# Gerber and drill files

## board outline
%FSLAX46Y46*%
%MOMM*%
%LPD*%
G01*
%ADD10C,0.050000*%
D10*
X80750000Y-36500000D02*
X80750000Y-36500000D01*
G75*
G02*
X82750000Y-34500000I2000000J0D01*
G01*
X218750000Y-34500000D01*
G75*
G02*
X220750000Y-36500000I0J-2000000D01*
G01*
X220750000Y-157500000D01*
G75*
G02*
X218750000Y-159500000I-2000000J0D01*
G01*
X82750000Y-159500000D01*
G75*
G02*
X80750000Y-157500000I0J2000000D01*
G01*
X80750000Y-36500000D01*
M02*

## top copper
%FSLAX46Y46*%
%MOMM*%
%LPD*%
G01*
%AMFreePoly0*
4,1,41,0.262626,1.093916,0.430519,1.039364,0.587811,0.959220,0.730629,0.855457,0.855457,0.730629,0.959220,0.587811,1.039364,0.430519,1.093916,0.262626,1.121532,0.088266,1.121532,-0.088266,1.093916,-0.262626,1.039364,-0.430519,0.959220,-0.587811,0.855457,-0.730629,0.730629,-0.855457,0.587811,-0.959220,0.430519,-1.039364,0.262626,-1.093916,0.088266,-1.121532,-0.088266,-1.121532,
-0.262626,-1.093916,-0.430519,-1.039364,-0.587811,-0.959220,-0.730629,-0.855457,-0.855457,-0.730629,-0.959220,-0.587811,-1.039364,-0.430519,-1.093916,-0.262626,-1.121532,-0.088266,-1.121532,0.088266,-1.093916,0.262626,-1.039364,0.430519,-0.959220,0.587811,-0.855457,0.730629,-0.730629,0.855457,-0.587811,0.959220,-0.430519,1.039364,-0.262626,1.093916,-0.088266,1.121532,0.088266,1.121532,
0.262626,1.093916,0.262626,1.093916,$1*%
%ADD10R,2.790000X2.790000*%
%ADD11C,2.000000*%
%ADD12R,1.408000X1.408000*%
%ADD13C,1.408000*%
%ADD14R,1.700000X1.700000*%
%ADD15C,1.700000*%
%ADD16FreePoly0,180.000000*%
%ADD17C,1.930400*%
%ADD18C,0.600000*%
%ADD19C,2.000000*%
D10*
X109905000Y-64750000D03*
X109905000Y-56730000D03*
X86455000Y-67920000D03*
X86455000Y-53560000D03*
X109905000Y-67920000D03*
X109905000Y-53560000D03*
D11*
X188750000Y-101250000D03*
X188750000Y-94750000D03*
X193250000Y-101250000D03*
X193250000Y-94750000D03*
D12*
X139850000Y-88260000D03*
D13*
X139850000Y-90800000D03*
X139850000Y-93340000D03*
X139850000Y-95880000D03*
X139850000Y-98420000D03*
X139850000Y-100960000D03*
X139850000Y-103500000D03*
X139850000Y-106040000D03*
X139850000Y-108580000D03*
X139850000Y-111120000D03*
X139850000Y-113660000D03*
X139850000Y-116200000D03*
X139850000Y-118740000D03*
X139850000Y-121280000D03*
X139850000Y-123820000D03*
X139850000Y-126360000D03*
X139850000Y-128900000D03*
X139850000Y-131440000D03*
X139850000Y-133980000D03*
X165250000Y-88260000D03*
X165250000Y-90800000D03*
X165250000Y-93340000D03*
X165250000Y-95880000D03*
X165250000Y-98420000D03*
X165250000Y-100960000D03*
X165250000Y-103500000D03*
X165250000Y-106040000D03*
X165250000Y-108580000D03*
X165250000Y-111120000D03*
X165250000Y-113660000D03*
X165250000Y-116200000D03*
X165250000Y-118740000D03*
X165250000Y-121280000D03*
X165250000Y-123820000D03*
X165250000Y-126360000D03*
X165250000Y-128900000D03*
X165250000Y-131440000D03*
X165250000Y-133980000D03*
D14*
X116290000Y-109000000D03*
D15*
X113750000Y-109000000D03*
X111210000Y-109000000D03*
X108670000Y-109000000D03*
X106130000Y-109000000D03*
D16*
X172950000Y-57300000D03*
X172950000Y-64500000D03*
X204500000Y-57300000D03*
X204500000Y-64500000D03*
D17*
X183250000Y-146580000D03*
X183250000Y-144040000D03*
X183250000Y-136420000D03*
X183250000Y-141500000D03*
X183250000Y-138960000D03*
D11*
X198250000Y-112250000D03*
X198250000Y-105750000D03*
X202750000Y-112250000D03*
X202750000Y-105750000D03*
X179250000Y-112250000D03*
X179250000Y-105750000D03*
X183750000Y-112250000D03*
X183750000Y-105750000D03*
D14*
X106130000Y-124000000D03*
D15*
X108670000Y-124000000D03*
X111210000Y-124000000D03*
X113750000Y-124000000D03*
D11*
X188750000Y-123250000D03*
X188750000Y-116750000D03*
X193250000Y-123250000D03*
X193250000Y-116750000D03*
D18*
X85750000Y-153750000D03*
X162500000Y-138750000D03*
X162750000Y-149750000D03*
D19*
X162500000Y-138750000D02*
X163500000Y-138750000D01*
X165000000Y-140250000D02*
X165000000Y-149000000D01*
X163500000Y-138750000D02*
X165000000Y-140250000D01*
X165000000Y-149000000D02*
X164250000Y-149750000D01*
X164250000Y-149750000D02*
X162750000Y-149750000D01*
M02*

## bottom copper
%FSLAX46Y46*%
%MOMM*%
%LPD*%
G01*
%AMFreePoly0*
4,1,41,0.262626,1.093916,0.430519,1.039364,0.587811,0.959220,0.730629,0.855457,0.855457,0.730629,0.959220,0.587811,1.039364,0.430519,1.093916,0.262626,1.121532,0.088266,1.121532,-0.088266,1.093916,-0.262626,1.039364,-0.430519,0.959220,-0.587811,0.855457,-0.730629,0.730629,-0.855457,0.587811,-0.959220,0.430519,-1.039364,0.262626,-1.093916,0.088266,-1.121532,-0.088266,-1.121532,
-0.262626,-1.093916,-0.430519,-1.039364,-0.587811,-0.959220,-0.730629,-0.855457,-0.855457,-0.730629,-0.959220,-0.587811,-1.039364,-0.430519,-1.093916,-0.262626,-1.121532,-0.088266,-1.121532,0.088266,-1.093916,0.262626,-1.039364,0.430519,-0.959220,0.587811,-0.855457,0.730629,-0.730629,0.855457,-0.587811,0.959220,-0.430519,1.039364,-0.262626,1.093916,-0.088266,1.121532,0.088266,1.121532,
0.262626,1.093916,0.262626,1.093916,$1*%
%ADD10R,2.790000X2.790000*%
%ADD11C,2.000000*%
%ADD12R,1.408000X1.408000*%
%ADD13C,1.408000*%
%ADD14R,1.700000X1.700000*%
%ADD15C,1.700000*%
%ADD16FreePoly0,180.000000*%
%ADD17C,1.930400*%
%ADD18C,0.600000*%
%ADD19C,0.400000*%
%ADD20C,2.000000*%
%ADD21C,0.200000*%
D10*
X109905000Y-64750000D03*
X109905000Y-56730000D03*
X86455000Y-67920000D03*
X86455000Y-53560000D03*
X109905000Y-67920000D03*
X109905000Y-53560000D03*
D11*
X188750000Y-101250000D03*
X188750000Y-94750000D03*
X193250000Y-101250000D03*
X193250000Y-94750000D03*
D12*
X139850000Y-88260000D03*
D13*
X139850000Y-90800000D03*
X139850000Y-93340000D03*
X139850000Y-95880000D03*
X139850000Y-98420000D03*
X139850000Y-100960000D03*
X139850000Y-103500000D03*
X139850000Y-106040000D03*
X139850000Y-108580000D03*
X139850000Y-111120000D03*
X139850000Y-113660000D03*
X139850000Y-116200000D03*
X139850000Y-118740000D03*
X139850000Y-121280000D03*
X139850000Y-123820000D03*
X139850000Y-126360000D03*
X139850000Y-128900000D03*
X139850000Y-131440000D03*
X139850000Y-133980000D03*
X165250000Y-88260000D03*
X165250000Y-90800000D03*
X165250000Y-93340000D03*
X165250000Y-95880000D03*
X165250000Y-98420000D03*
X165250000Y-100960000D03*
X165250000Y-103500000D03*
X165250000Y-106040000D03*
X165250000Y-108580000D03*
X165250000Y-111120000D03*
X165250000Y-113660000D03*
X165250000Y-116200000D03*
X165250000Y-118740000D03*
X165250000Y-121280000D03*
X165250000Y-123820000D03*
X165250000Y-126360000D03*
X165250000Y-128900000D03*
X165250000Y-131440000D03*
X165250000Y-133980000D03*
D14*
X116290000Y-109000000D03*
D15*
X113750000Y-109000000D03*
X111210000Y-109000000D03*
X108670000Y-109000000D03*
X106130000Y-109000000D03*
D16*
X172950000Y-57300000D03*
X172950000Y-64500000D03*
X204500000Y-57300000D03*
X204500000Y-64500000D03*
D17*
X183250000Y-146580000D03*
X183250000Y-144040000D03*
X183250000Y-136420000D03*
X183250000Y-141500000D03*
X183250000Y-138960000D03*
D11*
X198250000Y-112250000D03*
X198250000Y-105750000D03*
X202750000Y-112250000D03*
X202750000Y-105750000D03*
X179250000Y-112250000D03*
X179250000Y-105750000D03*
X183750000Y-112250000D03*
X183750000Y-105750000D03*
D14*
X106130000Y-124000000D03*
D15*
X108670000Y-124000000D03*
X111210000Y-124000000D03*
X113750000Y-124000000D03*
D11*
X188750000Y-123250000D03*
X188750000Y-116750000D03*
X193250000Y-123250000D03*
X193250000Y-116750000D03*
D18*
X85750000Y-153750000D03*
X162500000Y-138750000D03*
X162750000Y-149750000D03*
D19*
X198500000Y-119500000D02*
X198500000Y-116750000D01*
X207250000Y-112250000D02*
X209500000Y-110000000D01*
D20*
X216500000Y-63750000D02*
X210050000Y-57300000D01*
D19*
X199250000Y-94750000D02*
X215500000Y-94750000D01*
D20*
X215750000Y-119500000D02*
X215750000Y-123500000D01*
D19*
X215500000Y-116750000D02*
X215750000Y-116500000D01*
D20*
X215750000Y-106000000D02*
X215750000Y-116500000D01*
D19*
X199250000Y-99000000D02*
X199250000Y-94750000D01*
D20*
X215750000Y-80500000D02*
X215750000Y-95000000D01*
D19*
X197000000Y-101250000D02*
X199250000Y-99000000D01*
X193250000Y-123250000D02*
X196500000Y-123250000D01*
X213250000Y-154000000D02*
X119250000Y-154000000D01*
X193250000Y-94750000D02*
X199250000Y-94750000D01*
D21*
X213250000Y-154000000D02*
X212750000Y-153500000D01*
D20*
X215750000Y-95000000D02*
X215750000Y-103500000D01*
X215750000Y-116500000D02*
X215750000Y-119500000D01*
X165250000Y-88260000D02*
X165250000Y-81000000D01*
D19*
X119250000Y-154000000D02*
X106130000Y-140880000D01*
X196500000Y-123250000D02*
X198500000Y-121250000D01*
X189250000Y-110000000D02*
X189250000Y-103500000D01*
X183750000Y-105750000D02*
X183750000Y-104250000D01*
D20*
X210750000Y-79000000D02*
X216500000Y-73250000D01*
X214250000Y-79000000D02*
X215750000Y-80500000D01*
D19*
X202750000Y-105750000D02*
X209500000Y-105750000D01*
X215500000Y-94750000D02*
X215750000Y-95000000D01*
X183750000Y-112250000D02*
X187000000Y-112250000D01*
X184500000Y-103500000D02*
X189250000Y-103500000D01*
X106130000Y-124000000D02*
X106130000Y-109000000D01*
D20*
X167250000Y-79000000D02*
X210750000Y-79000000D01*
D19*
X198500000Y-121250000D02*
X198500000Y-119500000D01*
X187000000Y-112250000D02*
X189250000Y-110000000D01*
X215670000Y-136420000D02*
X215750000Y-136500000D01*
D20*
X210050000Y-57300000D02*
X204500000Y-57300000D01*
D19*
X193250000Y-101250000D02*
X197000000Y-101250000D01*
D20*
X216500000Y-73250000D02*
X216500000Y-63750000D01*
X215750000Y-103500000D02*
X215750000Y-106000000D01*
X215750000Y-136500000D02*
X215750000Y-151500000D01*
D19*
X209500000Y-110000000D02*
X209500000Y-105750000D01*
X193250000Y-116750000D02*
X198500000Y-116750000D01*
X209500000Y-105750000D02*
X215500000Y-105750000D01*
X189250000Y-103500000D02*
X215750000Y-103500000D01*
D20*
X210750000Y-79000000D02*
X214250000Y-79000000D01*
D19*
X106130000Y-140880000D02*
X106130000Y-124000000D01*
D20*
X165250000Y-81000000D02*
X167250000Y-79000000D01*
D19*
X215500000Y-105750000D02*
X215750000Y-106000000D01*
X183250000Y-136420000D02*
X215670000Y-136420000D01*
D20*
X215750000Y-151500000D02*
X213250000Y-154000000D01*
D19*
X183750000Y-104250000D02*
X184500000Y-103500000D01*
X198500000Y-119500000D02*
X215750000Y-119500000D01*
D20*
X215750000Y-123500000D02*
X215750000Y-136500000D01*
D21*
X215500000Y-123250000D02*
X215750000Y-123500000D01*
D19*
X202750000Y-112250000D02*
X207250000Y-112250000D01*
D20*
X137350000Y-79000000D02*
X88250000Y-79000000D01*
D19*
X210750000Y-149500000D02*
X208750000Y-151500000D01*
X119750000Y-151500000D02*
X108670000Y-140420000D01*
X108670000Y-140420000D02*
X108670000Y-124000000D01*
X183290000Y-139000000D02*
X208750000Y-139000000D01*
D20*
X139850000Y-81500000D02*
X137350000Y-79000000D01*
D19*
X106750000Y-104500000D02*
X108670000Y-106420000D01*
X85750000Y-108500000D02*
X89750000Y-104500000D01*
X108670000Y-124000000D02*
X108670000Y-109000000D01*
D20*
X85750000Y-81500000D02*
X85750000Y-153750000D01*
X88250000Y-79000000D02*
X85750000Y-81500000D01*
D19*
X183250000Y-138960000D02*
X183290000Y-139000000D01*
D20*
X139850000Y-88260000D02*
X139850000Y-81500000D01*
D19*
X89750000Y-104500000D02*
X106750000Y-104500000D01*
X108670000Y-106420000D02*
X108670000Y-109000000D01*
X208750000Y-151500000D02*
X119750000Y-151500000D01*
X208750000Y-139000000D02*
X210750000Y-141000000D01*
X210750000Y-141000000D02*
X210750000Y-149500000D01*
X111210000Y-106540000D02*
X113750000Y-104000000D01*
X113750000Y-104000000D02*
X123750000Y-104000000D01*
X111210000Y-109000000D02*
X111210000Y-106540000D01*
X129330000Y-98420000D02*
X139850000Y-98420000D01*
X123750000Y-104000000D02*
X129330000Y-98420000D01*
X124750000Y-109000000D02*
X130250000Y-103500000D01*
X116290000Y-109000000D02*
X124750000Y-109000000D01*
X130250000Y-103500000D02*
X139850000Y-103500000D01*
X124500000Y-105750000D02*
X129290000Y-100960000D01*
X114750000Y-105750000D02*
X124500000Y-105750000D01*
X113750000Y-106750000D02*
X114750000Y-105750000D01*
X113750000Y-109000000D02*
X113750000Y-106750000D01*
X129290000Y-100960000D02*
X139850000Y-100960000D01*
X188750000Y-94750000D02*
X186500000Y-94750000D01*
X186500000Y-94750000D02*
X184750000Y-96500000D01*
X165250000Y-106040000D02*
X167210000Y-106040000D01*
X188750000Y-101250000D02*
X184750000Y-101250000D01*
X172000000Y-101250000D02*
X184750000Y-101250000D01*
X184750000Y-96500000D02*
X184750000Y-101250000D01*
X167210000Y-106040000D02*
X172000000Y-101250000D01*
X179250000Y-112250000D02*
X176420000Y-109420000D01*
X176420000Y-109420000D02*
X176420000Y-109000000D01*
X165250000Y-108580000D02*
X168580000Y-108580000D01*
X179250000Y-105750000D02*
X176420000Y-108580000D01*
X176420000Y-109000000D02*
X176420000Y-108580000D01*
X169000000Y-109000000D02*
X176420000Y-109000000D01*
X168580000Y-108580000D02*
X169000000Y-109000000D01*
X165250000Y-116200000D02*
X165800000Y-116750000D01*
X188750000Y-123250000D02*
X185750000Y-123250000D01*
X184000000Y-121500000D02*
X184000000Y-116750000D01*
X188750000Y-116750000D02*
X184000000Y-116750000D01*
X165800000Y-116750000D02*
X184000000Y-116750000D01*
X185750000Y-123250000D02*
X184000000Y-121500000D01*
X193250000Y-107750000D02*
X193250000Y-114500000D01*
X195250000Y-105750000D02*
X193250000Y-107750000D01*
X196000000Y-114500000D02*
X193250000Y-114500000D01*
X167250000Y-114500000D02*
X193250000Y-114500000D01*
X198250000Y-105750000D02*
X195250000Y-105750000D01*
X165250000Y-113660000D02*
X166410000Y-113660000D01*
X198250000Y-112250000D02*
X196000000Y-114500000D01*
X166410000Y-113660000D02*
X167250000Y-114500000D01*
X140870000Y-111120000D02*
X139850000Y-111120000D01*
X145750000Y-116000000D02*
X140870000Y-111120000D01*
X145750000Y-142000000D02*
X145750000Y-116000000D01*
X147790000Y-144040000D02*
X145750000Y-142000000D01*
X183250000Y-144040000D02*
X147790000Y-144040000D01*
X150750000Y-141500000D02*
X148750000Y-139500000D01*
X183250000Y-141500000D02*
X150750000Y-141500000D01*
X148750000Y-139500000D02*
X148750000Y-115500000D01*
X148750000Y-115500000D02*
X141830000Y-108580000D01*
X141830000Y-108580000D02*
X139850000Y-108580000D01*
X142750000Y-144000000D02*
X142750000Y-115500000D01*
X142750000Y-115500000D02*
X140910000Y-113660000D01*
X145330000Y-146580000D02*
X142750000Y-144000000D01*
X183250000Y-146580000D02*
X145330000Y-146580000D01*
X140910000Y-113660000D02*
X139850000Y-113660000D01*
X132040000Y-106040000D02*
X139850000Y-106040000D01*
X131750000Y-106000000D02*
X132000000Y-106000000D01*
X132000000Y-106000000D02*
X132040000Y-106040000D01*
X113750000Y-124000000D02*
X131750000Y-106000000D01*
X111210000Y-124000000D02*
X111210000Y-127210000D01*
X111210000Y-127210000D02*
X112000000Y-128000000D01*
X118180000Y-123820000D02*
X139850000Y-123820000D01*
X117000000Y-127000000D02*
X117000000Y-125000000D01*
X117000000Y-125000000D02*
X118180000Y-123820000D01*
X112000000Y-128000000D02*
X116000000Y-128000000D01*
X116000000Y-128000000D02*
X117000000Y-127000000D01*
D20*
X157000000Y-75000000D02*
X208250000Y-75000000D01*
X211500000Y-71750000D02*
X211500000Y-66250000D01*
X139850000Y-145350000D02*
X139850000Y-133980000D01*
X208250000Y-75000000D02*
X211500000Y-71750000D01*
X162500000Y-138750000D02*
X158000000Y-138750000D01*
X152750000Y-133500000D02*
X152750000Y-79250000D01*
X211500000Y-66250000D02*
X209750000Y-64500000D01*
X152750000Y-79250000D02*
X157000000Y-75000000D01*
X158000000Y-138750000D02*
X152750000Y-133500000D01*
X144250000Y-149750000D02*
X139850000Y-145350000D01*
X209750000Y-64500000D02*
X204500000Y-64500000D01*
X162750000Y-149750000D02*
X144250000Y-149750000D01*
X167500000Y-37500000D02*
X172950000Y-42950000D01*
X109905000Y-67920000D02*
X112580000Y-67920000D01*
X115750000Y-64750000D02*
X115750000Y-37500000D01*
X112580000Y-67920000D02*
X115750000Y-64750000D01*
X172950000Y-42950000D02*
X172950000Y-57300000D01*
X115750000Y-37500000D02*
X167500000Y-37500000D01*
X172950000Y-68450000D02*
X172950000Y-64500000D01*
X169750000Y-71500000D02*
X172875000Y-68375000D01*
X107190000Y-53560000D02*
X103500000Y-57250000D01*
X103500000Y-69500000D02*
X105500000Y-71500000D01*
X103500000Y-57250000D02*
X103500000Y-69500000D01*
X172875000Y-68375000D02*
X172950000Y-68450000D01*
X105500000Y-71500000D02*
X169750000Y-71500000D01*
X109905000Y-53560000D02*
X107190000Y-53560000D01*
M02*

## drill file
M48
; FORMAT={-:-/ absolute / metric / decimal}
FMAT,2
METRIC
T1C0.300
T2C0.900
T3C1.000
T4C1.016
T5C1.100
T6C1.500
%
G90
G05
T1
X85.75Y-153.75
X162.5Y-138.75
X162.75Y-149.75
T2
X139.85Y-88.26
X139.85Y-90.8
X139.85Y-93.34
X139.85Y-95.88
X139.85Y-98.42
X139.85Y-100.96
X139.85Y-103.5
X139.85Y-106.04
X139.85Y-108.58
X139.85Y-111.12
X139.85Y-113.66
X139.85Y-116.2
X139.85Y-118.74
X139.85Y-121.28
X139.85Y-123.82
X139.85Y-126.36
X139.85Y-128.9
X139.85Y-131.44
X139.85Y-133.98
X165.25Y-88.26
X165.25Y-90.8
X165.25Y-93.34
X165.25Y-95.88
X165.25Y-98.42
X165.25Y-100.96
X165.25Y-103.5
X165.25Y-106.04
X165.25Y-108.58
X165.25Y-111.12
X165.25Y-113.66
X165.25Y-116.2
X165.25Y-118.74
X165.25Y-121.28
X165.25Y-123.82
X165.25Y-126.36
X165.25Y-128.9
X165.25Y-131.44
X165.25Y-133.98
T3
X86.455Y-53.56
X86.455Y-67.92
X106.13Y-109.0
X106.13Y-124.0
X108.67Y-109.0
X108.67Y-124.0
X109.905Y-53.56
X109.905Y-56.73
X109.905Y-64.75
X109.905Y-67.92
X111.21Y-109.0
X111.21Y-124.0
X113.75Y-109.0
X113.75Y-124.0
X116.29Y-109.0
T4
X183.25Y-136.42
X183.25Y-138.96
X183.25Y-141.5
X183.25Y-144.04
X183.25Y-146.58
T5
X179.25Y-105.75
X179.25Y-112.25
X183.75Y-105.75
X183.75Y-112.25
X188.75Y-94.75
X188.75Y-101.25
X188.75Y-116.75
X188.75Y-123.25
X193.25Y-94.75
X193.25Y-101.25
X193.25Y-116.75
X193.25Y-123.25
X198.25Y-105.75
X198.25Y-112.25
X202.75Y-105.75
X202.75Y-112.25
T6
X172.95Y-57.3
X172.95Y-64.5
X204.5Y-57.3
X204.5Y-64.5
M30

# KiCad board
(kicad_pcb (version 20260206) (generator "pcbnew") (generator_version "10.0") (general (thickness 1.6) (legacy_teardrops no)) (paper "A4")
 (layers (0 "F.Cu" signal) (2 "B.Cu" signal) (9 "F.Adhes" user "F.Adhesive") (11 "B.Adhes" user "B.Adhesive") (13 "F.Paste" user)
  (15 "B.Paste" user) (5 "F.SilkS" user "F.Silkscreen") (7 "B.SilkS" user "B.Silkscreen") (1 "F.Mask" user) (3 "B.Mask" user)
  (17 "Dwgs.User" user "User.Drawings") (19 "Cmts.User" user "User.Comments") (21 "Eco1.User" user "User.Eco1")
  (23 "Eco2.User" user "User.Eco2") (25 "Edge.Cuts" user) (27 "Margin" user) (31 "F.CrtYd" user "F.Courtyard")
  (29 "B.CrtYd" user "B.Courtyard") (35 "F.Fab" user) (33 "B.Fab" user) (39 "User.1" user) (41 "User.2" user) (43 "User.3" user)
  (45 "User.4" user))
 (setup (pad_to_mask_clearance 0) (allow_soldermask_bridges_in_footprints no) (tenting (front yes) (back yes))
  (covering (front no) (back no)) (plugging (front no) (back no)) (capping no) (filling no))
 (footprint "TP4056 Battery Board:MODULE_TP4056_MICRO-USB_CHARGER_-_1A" (layer "F.Cu") (at 98.18 60.74)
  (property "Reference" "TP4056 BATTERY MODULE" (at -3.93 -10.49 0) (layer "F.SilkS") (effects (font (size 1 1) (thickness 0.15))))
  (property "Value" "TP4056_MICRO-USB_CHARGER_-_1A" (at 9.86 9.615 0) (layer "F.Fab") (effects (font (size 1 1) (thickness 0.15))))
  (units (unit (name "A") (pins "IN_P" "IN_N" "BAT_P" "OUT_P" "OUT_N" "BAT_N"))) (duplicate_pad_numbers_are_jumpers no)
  (pad "BAT_N" thru_hole rect (at 11.725 4.01) (size 2.79 2.79) (drill 1) (layers "*.Cu" "*.Mask") (remove_unused_layers no)
   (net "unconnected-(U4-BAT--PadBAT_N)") (solder_mask_margin 0.102))
  (pad "BAT_P" thru_hole rect (at 11.725 -4.01) (size 2.79 2.79) (drill 1) (layers "*.Cu" "*.Mask") (remove_unused_layers no)
   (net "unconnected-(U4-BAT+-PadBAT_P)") (solder_mask_margin 0.102))
  (pad "IN_N" thru_hole rect (at -11.725 7.18) (size 2.79 2.79) (drill 1) (layers "*.Cu" "*.Mask") (remove_unused_layers no)
   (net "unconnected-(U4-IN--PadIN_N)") (solder_mask_margin 0.102))
  (pad "IN_P" thru_hole rect (at -11.725 -7.18) (size 2.79 2.79) (drill 1) (layers "*.Cu" "*.Mask") (remove_unused_layers no)
   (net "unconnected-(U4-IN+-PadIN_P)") (solder_mask_margin 0.102))
  (pad "OUT_N" thru_hole rect (at 11.725 7.18) (size 2.79 2.79) (drill 1) (layers "*.Cu" "*.Mask") (remove_unused_layers no)
   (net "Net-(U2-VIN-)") (solder_mask_margin 0.102))
  (pad "OUT_P" thru_hole rect (at 11.725 -7.18) (size 2.79 2.79) (drill 1) (layers "*.Cu" "*.Mask") (remove_unused_layers no)
   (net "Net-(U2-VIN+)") (solder_mask_margin 0.102)))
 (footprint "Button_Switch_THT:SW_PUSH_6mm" (layer "F.Cu") (at 188.75 101.25 90)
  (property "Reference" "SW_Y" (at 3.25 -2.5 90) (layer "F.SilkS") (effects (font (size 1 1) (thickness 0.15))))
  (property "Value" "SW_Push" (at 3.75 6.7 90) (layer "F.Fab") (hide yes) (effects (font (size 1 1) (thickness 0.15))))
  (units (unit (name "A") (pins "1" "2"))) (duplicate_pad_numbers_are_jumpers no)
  (pad "1" thru_hole circle (at 0 0 180) (size 2 2) (drill 1.1) (layers "*.Cu" "*.Mask") (remove_unused_layers no) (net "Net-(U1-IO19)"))
  (pad "1" thru_hole circle (at 6.5 0 180) (size 2 2) (drill 1.1) (layers "*.Cu" "*.Mask") (remove_unused_layers no) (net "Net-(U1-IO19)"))
  (pad "2" thru_hole circle (at 0 4.5 180) (size 2 2) (drill 1.1) (layers "*.Cu" "*.Mask") (remove_unused_layers no) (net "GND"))
  (pad "2" thru_hole circle (at 6.5 4.5 180) (size 2 2) (drill 1.1) (layers "*.Cu" "*.Mask") (remove_unused_layers no) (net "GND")))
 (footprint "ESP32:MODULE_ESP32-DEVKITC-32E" (layer "F.Cu") (at 152.55 111.095)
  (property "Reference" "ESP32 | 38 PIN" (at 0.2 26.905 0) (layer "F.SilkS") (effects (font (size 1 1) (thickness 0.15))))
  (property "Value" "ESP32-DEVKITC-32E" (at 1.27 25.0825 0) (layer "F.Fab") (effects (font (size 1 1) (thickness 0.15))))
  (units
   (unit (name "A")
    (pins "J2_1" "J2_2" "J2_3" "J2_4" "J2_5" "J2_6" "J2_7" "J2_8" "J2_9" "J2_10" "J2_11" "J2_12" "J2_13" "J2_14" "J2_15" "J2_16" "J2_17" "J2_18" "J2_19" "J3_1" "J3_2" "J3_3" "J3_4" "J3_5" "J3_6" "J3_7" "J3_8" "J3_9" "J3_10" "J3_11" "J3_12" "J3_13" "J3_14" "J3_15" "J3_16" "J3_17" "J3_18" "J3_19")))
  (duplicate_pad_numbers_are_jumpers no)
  (pad "J2_1" thru_hole rect (at -12.7 -22.835) (size 1.408 1.408) (drill 0.9) (layers "*.Cu" "*.Mask") (remove_unused_layers no)
   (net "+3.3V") (solder_mask_margin 0.102))
  (pad "J2_2" thru_hole circle (at -12.7 -20.295) (size 1.408 1.408) (drill 0.9) (layers "*.Cu" "*.Mask") (remove_unused_layers no)
   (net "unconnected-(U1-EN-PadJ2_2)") (solder_mask_margin 0.102))
  (pad "J2_3" thru_hole circle (at -12.7 -17.755) (size 1.408 1.408) (drill 0.9) (layers "*.Cu" "*.Mask") (remove_unused_layers no)
   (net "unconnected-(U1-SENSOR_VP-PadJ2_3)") (solder_mask_margin 0.102))
  (pad "J2_4" thru_hole circle (at -12.7 -15.215) (size 1.408 1.408) (drill oval 0.9) (layers "*.Cu" "*.Mask") (remove_unused_layers no)
   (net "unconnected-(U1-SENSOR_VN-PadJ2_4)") (solder_mask_margin 0.102))
  (pad "J2_5" thru_hole circle (at -12.7 -12.675) (size 1.408 1.408) (drill 0.9) (layers "*.Cu" "*.Mask") (remove_unused_layers no)
   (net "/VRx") (solder_mask_margin 0.102))
  (pad "J2_6" thru_hole circle (at -12.7 -10.135) (size 1.408 1.408) (drill 0.9) (layers "*.Cu" "*.Mask") (remove_unused_layers no)
   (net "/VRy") (solder_mask_margin 0.102))
  (pad "J2_7" thru_hole circle (at -12.7 -7.595) (size 1.408 1.408) (drill 0.9) (layers "*.Cu" "*.Mask") (remove_unused_layers no)
   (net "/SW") (solder_mask_margin 0.102))
  (pad "J2_8" thru_hole circle (at -12.7 -5.055) (size 1.408 1.408) (drill 0.9) (layers "*.Cu" "*.Mask") (remove_unused_layers no)
   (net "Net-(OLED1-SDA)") (solder_mask_margin 0.102))
  (pad "J2_9" thru_hole circle (at -12.7 -2.515) (size 1.408 1.408) (drill 0.9) (layers "*.Cu" "*.Mask") (remove_unused_layers no)
   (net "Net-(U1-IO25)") (solder_mask_margin 0.102))
  (pad "J2_10" thru_hole circle (at -12.7 0.025) (size 1.408 1.408) (drill 0.9) (layers "*.Cu" "*.Mask") (remove_unused_layers no)
   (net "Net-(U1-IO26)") (solder_mask_margin 0.102))
  (pad "J2_11" thru_hole circle (at -12.7 2.565) (size 1.408 1.408) (drill 0.9) (layers "*.Cu" "*.Mask") (remove_unused_layers no)
   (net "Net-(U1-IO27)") (solder_mask_margin 0.102))
  (pad "J2_12" thru_hole circle (at -12.7 5.105) (size 1.408 1.408) (drill 0.9) (layers "*.Cu" "*.Mask") (remove_unused_layers no)
   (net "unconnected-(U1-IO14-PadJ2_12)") (solder_mask_margin 0.102))
  (pad "J2_13" thru_hole circle (at -12.7 7.645) (size 1.408 1.408) (drill 0.9) (layers "*.Cu" "*.Mask") (remove_unused_layers no)
   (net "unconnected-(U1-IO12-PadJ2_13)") (solder_mask_margin 0.102))
  (pad "J2_14" thru_hole circle (at -12.7 10.185) (size 1.408 1.408) (drill 0.9) (layers "*.Cu" "*.Mask") (remove_unused_layers no)
   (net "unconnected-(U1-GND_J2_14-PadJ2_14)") (solder_mask_margin 0.102))
  (pad "J2_15" thru_hole circle (at -12.7 12.725) (size 1.408 1.408) (drill 0.9) (layers "*.Cu" "*.Mask") (remove_unused_layers no)
   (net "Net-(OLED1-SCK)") (solder_mask_margin 0.102))
  (pad "J2_16" thru_hole circle (at -12.7 15.265) (size 1.408 1.408) (drill 0.9) (layers "*.Cu" "*.Mask") (remove_unused_layers no)
   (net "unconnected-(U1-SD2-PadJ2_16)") (solder_mask_margin 0.102))
  (pad "J2_17" thru_hole circle (at -12.7 17.805) (size 1.408 1.408) (drill 0.9) (layers "*.Cu" "*.Mask") (remove_unused_layers no)
   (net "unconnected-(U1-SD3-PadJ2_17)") (solder_mask_margin 0.102))
  (pad "J2_18" thru_hole circle (at -12.7 20.345) (size 1.408 1.408) (drill 0.9) (layers "*.Cu" "*.Mask") (remove_unused_layers no)
   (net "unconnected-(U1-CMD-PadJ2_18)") (solder_mask_margin 0.102))
  (pad "J2_19" thru_hole circle (at -12.7 22.885) (size 1.408 1.408) (drill 0.9) (layers "*.Cu" "*.Mask") (remove_unused_layers no)
   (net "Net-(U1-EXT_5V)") (solder_mask_margin 0.102))
  (pad "J3_1" thru_hole circle (at 12.7 -22.835) (size 1.408 1.408) (drill 0.9) (layers "*.Cu" "*.Mask") (remove_unused_layers no)
   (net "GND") (solder_mask_margin 0.102))
  (pad "J3_2" thru_hole circle (at 12.7 -20.295) (size 1.408 1.408) (drill 0.9) (layers "*.Cu" "*.Mask") (remove_unused_layers no)
   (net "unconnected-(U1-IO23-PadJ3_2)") (solder_mask_margin 0.102))
  (pad "J3_3" thru_hole circle (at 12.7 -17.755) (size 1.408 1.408) (drill 0.9) (layers "*.Cu" "*.Mask") (remove_unused_layers no)
   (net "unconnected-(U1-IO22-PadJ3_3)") (solder_mask_margin 0.102))
  (pad "J3_4" thru_hole circle (at 12.7 -15.215) (size 1.408 1.408) (drill 0.9) (layers "*.Cu" "*.Mask") (remove_unused_layers no)
   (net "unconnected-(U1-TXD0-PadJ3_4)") (solder_mask_margin 0.102))
  (pad "J3_5" thru_hole circle (at 12.7 -12.675) (size 1.408 1.408) (drill 0.9) (layers "*.Cu" "*.Mask") (remove_unused_layers no)
   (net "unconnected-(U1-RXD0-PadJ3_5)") (solder_mask_margin 0.102))
  (pad "J3_6" thru_hole circle (at 12.7 -10.135) (size 1.408 1.408) (drill 0.9) (layers "*.Cu" "*.Mask") (remove_unused_layers no)
   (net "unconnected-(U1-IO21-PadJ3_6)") (solder_mask_margin 0.102))
  (pad "J3_7" thru_hole circle (at 12.7 -7.595) (size 1.408 1.408) (drill 0.9) (layers "*.Cu" "*.Mask") (remove_unused_layers no)
   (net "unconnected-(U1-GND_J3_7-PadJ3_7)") (solder_mask_margin 0.102))
  (pad "J3_8" thru_hole circle (at 12.7 -5.055) (size 1.408 1.408) (drill 0.9) (layers "*.Cu" "*.Mask") (remove_unused_layers no)
   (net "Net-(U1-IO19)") (solder_mask_margin 0.102))
  (pad "J3_9" thru_hole circle (at 12.7 -2.515) (size 1.408 1.408) (drill 0.9) (layers "*.Cu" "*.Mask") (remove_unused_layers no)
   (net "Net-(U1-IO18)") (solder_mask_margin 0.102))
  (pad "J3_10" thru_hole circle (at 12.7 0.025) (size 1.408 1.408) (drill 0.9) (layers "*.Cu" "*.Mask") (remove_unused_layers no)
   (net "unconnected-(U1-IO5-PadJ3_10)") (solder_mask_margin 0.102))
  (pad "J3_11" thru_hole circle (at 12.7 2.565) (size 1.408 1.408) (drill 0.9) (layers "*.Cu" "*.Mask") (remove_unused_layers no)
   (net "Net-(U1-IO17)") (solder_mask_margin 0.102))
  (pad "J3_12" thru_hole circle (at 12.7 5.105) (size 1.408 1.408) (drill 0.9) (layers "*.Cu" "*.Mask") (remove_unused_layers no)
   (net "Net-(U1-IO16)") (solder_mask_margin 0.102))
  (pad "J3_13" thru_hole circle (at 12.7 7.645) (size 1.408 1.408) (drill 0.9) (layers "*.Cu" "*.Mask") (remove_unused_layers no)
   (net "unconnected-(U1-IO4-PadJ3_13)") (solder_mask_margin 0.102))
  (pad "J3_14" thru_hole circle (at 12.7 10.185) (size 1.408 1.408) (drill 0.9) (layers "*.Cu" "*.Mask") (remove_unused_layers no)
   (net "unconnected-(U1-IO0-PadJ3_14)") (solder_mask_margin 0.102))
  (pad "J3_15" thru_hole circle (at 12.7 12.725) (size 1.408 1.408) (drill 0.9) (layers "*.Cu" "*.Mask") (remove_unused_layers no)
   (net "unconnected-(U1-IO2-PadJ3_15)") (solder_mask_margin 0.102))
  (pad "J3_16" thru_hole circle (at 12.7 15.265) (size 1.408 1.408) (drill 0.9) (layers "*.Cu" "*.Mask") (remove_unused_layers no)
   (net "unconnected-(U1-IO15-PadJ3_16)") (solder_mask_margin 0.102))
  (pad "J3_17" thru_hole circle (at 12.7 17.805) (size 1.408 1.408) (drill 0.9) (layers "*.Cu" "*.Mask") (remove_unused_layers no)
   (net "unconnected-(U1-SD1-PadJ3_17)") (solder_mask_margin 0.102))
  (pad "J3_18" thru_hole circle (at 12.7 20.345) (size 1.408 1.408) (drill 0.9) (layers "*.Cu" "*.Mask") (remove_unused_layers no)
   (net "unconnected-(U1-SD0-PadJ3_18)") (solder_mask_margin 0.102))
  (pad "J3_19" thru_hole circle (at 12.7 22.885) (size 1.408 1.408) (drill 0.9) (layers "*.Cu" "*.Mask") (remove_unused_layers no)
   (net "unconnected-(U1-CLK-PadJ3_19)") (solder_mask_margin 0.102)))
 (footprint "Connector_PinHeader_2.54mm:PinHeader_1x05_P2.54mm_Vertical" (layer "F.Cu") (at 116.29 109 -90)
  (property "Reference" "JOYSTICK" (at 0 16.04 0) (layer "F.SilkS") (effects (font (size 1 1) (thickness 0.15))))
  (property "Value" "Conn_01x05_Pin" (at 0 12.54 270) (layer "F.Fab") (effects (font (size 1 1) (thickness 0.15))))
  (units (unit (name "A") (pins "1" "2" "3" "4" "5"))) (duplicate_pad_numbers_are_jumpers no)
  (pad "1" thru_hole rect (at 0 0 270) (size 1.7 1.7) (drill 1) (layers "*.Cu" "*.Mask") (remove_unused_layers no) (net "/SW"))
  (pad "2" thru_hole circle (at 0 2.54 270) (size 1.7 1.7) (drill 1) (layers "*.Cu" "*.Mask") (remove_unused_layers no) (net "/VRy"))
  (pad "3" thru_hole circle (at 0 5.08 270) (size 1.7 1.7) (drill 1) (layers "*.Cu" "*.Mask") (remove_unused_layers no) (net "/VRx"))
  (pad "4" thru_hole circle (at 0 7.62 270) (size 1.7 1.7) (drill 1) (layers "*.Cu" "*.Mask") (remove_unused_layers no) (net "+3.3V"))
  (pad "5" thru_hole circle (at 0 10.16 270) (size 1.7 1.7) (drill 1) (layers "*.Cu" "*.Mask") (remove_unused_layers no) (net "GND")))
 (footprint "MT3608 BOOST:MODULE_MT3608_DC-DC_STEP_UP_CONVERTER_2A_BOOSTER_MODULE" (layer "F.Cu") (at 188.725 60.9 180)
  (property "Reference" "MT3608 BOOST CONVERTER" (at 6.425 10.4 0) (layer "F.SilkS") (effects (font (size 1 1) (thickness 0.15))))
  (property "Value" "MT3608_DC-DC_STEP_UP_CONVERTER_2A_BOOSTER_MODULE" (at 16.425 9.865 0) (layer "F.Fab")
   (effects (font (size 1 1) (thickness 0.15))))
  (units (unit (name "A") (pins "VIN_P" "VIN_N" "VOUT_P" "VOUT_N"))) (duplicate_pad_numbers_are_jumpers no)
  (pad "VIN_N" thru_hole custom (at 15.775 3.6 180) (size 2.25 2.25) (drill 1.5) (layers "*.Cu") (remove_unused_layers no)
   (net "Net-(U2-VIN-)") (thermal_bridge_angle 90) (options (clearance outline) (anchor circle)) (primitives))
  (pad "VIN_P" thru_hole custom (at 15.775 -3.6 180) (size 2.25 2.25) (drill 1.5) (layers "*.Cu") (remove_unused_layers no)
   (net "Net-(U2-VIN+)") (thermal_bridge_angle 90) (options (clearance outline) (anchor circle)) (primitives))
  (pad "VOUT_N" thru_hole custom (at -15.775 3.6 180) (size 2.25 2.25) (drill 1.5) (layers "*.Cu") (remove_unused_layers no) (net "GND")
   (thermal_bridge_angle 90) (options (clearance outline) (anchor circle)) (primitives))
  (pad "VOUT_P" thru_hole custom (at -15.775 -3.6 180) (size 2.25 2.25) (drill 1.5) (layers "*.Cu") (remove_unused_layers no)
   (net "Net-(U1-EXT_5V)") (thermal_bridge_angle 90) (options (clearance outline) (anchor circle)) (primitives)))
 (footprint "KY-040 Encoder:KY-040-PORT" (layer "F.Cu") (at 183.25 140.23 90)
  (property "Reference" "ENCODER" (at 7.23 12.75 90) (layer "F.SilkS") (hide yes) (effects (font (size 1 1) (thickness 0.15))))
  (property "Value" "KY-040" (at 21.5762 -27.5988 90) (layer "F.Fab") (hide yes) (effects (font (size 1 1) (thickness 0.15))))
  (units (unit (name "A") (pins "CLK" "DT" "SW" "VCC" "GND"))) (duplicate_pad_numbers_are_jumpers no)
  (pad "CLK" thru_hole circle (at -6.35 0 90) (size 1.9304 1.9304) (drill 1.016) (layers "*.Cu" "*.Mask") (remove_unused_layers no)
   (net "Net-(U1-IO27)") (solder_mask_margin 0.102))
  (pad "DT" thru_hole circle (at -3.81 0 90) (size 1.9304 1.9304) (drill 1.016) (layers "*.Cu" "*.Mask") (remove_unused_layers no)
   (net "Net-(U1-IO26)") (solder_mask_margin 0.102))
  (pad "GND" thru_hole circle (at 3.81 0 90) (size 1.9304 1.9304) (drill 1.016) (layers "*.Cu" "*.Mask") (remove_unused_layers no)
   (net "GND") (solder_mask_margin 0.102))
  (pad "SW" thru_hole circle (at -1.27 0 90) (size 1.9304 1.9304) (drill 1.016) (layers "*.Cu" "*.Mask") (remove_unused_layers no)
   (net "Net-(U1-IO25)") (solder_mask_margin 0.102))
  (pad "VCC" thru_hole circle (at 1.27 0 90) (size 1.9304 1.9304) (drill 1.016) (layers "*.Cu" "*.Mask") (remove_unused_layers no)
   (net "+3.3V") (solder_mask_margin 0.102)))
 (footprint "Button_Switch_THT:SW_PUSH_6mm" (layer "F.Cu") (at 198.25 112.25 90)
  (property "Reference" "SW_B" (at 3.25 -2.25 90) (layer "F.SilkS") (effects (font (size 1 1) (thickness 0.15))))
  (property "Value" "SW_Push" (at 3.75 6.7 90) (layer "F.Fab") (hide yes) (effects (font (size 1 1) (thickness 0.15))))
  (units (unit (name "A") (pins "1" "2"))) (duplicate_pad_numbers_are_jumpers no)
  (pad "1" thru_hole circle (at 0 0 180) (size 2 2) (drill 1.1) (layers "*.Cu" "*.Mask") (remove_unused_layers no) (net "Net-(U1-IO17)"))
  (pad "1" thru_hole circle (at 6.5 0 180) (size 2 2) (drill 1.1) (layers "*.Cu" "*.Mask") (remove_unused_layers no) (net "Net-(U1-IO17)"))
  (pad "2" thru_hole circle (at 0 4.5 180) (size 2 2) (drill 1.1) (layers "*.Cu" "*.Mask") (remove_unused_layers no) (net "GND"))
  (pad "2" thru_hole circle (at 6.5 4.5 180) (size 2 2) (drill 1.1) (layers "*.Cu" "*.Mask") (remove_unused_layers no) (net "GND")))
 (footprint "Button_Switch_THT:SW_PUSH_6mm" (layer "F.Cu") (at 179.25 112.25 90)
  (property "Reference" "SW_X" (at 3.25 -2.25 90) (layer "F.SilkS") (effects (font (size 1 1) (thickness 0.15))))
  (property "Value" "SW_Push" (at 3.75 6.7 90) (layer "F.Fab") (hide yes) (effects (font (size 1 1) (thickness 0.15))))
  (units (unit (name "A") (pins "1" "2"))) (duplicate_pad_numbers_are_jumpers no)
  (pad "1" thru_hole circle (at 0 0 180) (size 2 2) (drill 1.1) (layers "*.Cu" "*.Mask") (remove_unused_layers no) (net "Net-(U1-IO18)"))
  (pad "1" thru_hole circle (at 6.5 0 180) (size 2 2) (drill 1.1) (layers "*.Cu" "*.Mask") (remove_unused_layers no) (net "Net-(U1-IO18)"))
  (pad "2" thru_hole circle (at 0 4.5 180) (size 2 2) (drill 1.1) (layers "*.Cu" "*.Mask") (remove_unused_layers no) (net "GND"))
  (pad "2" thru_hole circle (at 6.5 4.5 180) (size 2 2) (drill 1.1) (layers "*.Cu" "*.Mask") (remove_unused_layers no) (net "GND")))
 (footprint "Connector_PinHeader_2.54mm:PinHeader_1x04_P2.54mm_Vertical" (layer "F.Cu") (at 106.13 124 90)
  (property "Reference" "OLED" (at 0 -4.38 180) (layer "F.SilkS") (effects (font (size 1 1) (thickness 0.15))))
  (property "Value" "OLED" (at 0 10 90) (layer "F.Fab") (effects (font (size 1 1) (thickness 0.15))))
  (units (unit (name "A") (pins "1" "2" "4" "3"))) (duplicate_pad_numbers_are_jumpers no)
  (pad "1" thru_hole rect (at 0 0 90) (size 1.7 1.7) (drill 1) (layers "*.Cu" "*.Mask") (remove_unused_layers no) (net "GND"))
  (pad "2" thru_hole circle (at 0 2.54 90) (size 1.7 1.7) (drill 1) (layers "*.Cu" "*.Mask") (remove_unused_layers no) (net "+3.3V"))
  (pad "3" thru_hole circle (at 0 5.08 90) (size 1.7 1.7) (drill 1) (layers "*.Cu" "*.Mask") (remove_unused_layers no)
   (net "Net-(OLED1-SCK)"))
  (pad "4" thru_hole circle (at 0 7.62 90) (size 1.7 1.7) (drill 1) (layers "*.Cu" "*.Mask") (remove_unused_layers no)
   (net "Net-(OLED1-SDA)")))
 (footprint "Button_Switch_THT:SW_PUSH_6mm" (layer "F.Cu") (at 188.75 123.25 90)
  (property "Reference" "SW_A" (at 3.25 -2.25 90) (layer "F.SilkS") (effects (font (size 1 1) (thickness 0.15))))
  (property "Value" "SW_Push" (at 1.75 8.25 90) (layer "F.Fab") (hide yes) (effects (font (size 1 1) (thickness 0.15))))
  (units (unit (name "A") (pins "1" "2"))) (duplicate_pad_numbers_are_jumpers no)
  (pad "1" thru_hole circle (at 0 0 180) (size 2 2) (drill 1.1) (layers "*.Cu" "*.Mask") (remove_unused_layers no) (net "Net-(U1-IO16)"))
  (pad "1" thru_hole circle (at 6.5 0 180) (size 2 2) (drill 1.1) (layers "*.Cu" "*.Mask") (remove_unused_layers no) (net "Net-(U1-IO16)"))
  (pad "2" thru_hole circle (at 0 4.5 180) (size 2 2) (drill 1.1) (layers "*.Cu" "*.Mask") (remove_unused_layers no) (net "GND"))
  (pad "2" thru_hole circle (at 6.5 4.5 180) (size 2 2) (drill 1.1) (layers "*.Cu" "*.Mask") (remove_unused_layers no) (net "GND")))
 (gr_rect (start 80.75 34.5) (end 220.75 159.5) (radius 2) (stroke (width 0.05) (type solid)) (fill no) (layer "Edge.Cuts"))
 (segment (start 198.5 119.5) (end 198.5 116.75) (width 0.4) (layer "B.Cu") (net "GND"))
 (segment (start 207.25 112.25) (end 209.5 110) (width 0.4) (layer "B.Cu") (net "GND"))
 (segment (start 216.5 63.75) (end 210.05 57.3) (width 2) (layer "B.Cu") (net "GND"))
 (segment (start 199.25 94.75) (end 215.5 94.75) (width 0.4) (layer "B.Cu") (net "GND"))
 (segment (start 215.75 119.5) (end 215.75 123.5) (width 2) (layer "B.Cu") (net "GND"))
 (segment (start 215.5 116.75) (end 215.75 116.5) (width 0.4) (layer "B.Cu") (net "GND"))
 (segment (start 215.75 106) (end 215.75 116.5) (width 2) (layer "B.Cu") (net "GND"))
 (segment (start 199.25 99) (end 199.25 94.75) (width 0.4) (layer "B.Cu") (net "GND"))
 (segment (start 215.75 80.5) (end 215.75 95) (width 2) (layer "B.Cu") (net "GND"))
 (segment (start 197 101.25) (end 199.25 99) (width 0.4) (layer "B.Cu") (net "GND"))
 (segment (start 193.25 123.25) (end 196.5 123.25) (width 0.4) (layer "B.Cu") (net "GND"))
 (segment (start 213.25 154) (end 119.25 154) (width 0.4) (layer "B.Cu") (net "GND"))
 (segment (start 193.25 94.75) (end 199.25 94.75) (width 0.4) (layer "B.Cu") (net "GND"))
 (segment (start 213.25 154) (end 212.75 153.5) (width 0.2) (layer "B.Cu") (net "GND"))
 (segment (start 215.75 95) (end 215.75 103.5) (width 2) (layer "B.Cu") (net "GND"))
 (segment (start 215.75 116.5) (end 215.75 119.5) (width 2) (layer "B.Cu") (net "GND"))
 (segment (start 165.25 88.26) (end 165.25 81) (width 2) (layer "B.Cu") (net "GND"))
 (segment (start 119.25 154) (end 106.13 140.88) (width 0.4) (layer "B.Cu") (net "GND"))
 (segment (start 196.5 123.25) (end 198.5 121.25) (width 0.4) (layer "B.Cu") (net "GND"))
 (segment (start 189.25 110) (end 189.25 103.5) (width 0.4) (layer "B.Cu") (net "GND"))
 (segment (start 183.75 105.75) (end 183.75 104.25) (width 0.4) (layer "B.Cu") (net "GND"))
 (segment (start 210.75 79) (end 216.5 73.25) (width 2) (layer "B.Cu") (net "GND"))
 (segment (start 214.25 79) (end 215.75 80.5) (width 2) (layer "B.Cu") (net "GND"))
 (segment (start 202.75 105.75) (end 209.5 105.75) (width 0.4) (layer "B.Cu") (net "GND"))
 (segment (start 215.5 94.75) (end 215.75 95) (width 0.4) (layer "B.Cu") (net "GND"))
 (segment (start 183.75 112.25) (end 187 112.25) (width 0.4) (layer "B.Cu") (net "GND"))
 (segment (start 184.5 103.5) (end 189.25 103.5) (width 0.4) (layer "B.Cu") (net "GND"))
 (segment (start 106.13 124) (end 106.13 109) (width 0.4) (layer "B.Cu") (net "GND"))
 (segment (start 167.25 79) (end 210.75 79) (width 2) (layer "B.Cu") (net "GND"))
 (segment (start 198.5 121.25) (end 198.5 119.5) (width 0.4) (layer "B.Cu") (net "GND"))
 (segment (start 187 112.25) (end 189.25 110) (width 0.4) (layer "B.Cu") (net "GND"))
 (segment (start 215.67 136.42) (end 215.75 136.5) (width 0.4) (layer "B.Cu") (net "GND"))
 (segment (start 210.05 57.3) (end 204.5 57.3) (width 2) (layer "B.Cu") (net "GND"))
 (segment (start 193.25 101.25) (end 197 101.25) (width 0.4) (layer "B.Cu") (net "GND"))
 (segment (start 216.5 73.25) (end 216.5 63.75) (width 2) (layer "B.Cu") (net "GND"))
 (segment (start 215.75 103.5) (end 215.75 106) (width 2) (layer "B.Cu") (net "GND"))
 (segment (start 215.75 136.5) (end 215.75 151.5) (width 2) (layer "B.Cu") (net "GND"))
 (segment (start 209.5 110) (end 209.5 105.75) (width 0.4) (layer "B.Cu") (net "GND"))
 (segment (start 193.25 116.75) (end 198.5 116.75) (width 0.4) (layer "B.Cu") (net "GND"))
 (segment (start 209.5 105.75) (end 215.5 105.75) (width 0.4) (layer "B.Cu") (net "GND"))
 (segment (start 189.25 103.5) (end 215.75 103.5) (width 0.4) (layer "B.Cu") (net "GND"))
 (segment (start 210.75 79) (end 214.25 79) (width 2) (layer "B.Cu") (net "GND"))
 (segment (start 106.13 140.88) (end 106.13 124) (width 0.4) (layer "B.Cu") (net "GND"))
 (segment (start 165.25 81) (end 167.25 79) (width 2) (layer "B.Cu") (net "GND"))
 (segment (start 215.5 105.75) (end 215.75 106) (width 0.4) (layer "B.Cu") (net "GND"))
 (segment (start 183.25 136.42) (end 215.67 136.42) (width 0.4) (layer "B.Cu") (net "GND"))
 (segment (start 215.75 151.5) (end 213.25 154) (width 2) (layer "B.Cu") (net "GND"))
 (segment (start 183.75 104.25) (end 184.5 103.5) (width 0.4) (layer "B.Cu") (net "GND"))
 (segment (start 198.5 119.5) (end 215.75 119.5) (width 0.4) (layer "B.Cu") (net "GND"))
 (segment (start 215.75 123.5) (end 215.75 136.5) (width 2) (layer "B.Cu") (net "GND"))
 (segment (start 215.5 123.25) (end 215.75 123.5) (width 0.2) (layer "B.Cu") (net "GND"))
 (segment (start 202.75 112.25) (end 207.25 112.25) (width 0.4) (layer "B.Cu") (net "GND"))
 (via (at 85.75 153.75) (size 0.6) (drill 0.3) (layers "F.Cu" "B.Cu") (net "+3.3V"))
 (segment (start 137.35 79) (end 88.25 79) (width 2) (layer "B.Cu") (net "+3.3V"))
 (segment (start 210.75 149.5) (end 208.75 151.5) (width 0.4) (layer "B.Cu") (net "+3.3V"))
 (segment (start 119.75 151.5) (end 108.67 140.42) (width 0.4) (layer "B.Cu") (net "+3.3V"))
 (segment (start 108.67 140.42) (end 108.67 124) (width 0.4) (layer "B.Cu") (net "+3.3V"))
 (segment (start 183.29 139) (end 208.75 139) (width 0.4) (layer "B.Cu") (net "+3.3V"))
 (segment (start 139.85 81.5) (end 137.35 79) (width 2) (layer "B.Cu") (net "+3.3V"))
 (segment (start 106.75 104.5) (end 108.67 106.42) (width 0.4) (layer "B.Cu") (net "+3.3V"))
 (segment (start 85.75 108.5) (end 89.75 104.5) (width 0.4) (layer "B.Cu") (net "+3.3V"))
 (segment (start 108.67 124) (end 108.67 109) (width 0.4) (layer "B.Cu") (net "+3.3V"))
 (segment (start 85.75 81.5) (end 85.75 153.75) (width 2) (layer "B.Cu") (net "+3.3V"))
 (segment (start 88.25 79) (end 85.75 81.5) (width 2) (layer "B.Cu") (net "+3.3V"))
 (segment (start 183.25 138.96) (end 183.29 139) (width 0.4) (layer "B.Cu") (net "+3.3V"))
 (segment (start 139.85 88.26) (end 139.85 81.5) (width 2) (layer "B.Cu") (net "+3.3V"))
 (segment (start 89.75 104.5) (end 106.75 104.5) (width 0.4) (layer "B.Cu") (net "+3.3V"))
 (segment (start 108.67 106.42) (end 108.67 109) (width 0.4) (layer "B.Cu") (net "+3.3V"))
 (segment (start 208.75 151.5) (end 119.75 151.5) (width 0.4) (layer "B.Cu") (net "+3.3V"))
 (segment (start 208.75 139) (end 210.75 141) (width 0.4) (layer "B.Cu") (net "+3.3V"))
 (segment (start 210.75 141) (end 210.75 149.5) (width 0.4) (layer "B.Cu") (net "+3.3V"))
 (segment (start 111.21 106.54) (end 113.75 104) (width 0.4) (layer "B.Cu") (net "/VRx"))
 (segment (start 113.75 104) (end 123.75 104) (width 0.4) (layer "B.Cu") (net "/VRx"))
 (segment (start 111.21 109) (end 111.21 106.54) (width 0.4) (layer "B.Cu") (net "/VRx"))
 (segment (start 129.33 98.42) (end 139.85 98.42) (width 0.4) (layer "B.Cu") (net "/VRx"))
 (segment (start 123.75 104) (end 129.33 98.42) (width 0.4) (layer "B.Cu") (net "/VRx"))
 (segment (start 124.75 109) (end 130.25 103.5) (width 0.4) (layer "B.Cu") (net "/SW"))
 (segment (start 116.29 109) (end 124.75 109) (width 0.4) (layer "B.Cu") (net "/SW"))
 (segment (start 130.25 103.5) (end 139.85 103.5) (width 0.4) (layer "B.Cu") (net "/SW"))
 (segment (start 124.5 105.75) (end 129.29 100.96) (width 0.4) (layer "B.Cu") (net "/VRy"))
 (segment (start 114.75 105.75) (end 124.5 105.75) (width 0.4) (layer "B.Cu") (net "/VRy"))
 (segment (start 113.75 106.75) (end 114.75 105.75) (width 0.4) (layer "B.Cu") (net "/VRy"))
 (segment (start 113.75 109) (end 113.75 106.75) (width 0.4) (layer "B.Cu") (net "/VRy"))
 (segment (start 129.29 100.96) (end 139.85 100.96) (width 0.4) (layer "B.Cu") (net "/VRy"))
 (segment (start 188.75 94.75) (end 186.5 94.75) (width 0.4) (layer "B.Cu") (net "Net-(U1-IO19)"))
 (segment (start 186.5 94.75) (end 184.75 96.5) (width 0.4) (layer "B.Cu") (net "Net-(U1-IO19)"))
 (segment (start 165.25 106.04) (end 167.21 106.04) (width 0.4) (layer "B.Cu") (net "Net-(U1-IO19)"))
 (segment (start 188.75 101.25) (end 184.75 101.25) (width 0.4) (layer "B.Cu") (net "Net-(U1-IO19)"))
 (segment (start 172 101.25) (end 184.75 101.25) (width 0.4) (layer "B.Cu") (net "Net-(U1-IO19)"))
 (segment (start 184.75 96.5) (end 184.75 101.25) (width 0.4) (layer "B.Cu") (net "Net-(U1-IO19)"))
 (segment (start 167.21 106.04) (end 172 101.25) (width 0.4) (layer "B.Cu") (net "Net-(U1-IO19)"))
 (segment (start 179.25 112.25) (end 176.42 109.42) (width 0.4) (layer "B.Cu") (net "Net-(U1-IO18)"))
 (segment (start 176.42 109.42) (end 176.42 109) (width 0.4) (layer "B.Cu") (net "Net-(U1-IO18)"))
 (segment (start 165.25 108.58) (end 168.58 108.58) (width 0.4) (layer "B.Cu") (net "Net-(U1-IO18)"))
 (segment (start 179.25 105.75) (end 176.42 108.58) (width 0.4) (layer "B.Cu") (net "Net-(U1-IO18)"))
 (segment (start 176.42 109) (end 176.42 108.58) (width 0.4) (layer "B.Cu") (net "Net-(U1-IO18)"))
 (segment (start 169 109) (end 176.42 109) (width 0.4) (layer "B.Cu") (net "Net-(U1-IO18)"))
 (segment (start 168.58 108.58) (end 169 109) (width 0.4) (layer "B.Cu") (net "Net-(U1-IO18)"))
 (segment (start 165.25 116.2) (end 165.8 116.75) (width 0.4) (layer "B.Cu") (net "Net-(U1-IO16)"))
 (segment (start 188.75 123.25) (end 185.75 123.25) (width 0.4) (layer "B.Cu") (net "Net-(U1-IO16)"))
 (segment (start 184 121.5) (end 184 116.75) (width 0.4) (layer "B.Cu") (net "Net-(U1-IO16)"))
 (segment (start 188.75 116.75) (end 184 116.75) (width 0.4) (layer "B.Cu") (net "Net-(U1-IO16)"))
 (segment (start 165.8 116.75) (end 184 116.75) (width 0.4) (layer "B.Cu") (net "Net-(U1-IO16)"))
 (segment (start 185.75 123.25) (end 184 121.5) (width 0.4) (layer "B.Cu") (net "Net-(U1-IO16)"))
 (segment (start 193.25 107.75) (end 193.25 114.5) (width 0.4) (layer "B.Cu") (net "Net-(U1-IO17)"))
 (segment (start 195.25 105.75) (end 193.25 107.75) (width 0.4) (layer "B.Cu") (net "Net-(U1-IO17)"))
 (segment (start 196 114.5) (end 193.25 114.5) (width 0.4) (layer "B.Cu") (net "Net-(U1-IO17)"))
 (segment (start 167.25 114.5) (end 193.25 114.5) (width 0.4) (layer "B.Cu") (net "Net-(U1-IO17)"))
 (segment (start 198.25 105.75) (end 195.25 105.75) (width 0.4) (layer "B.Cu") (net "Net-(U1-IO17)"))
 (segment (start 165.25 113.66) (end 166.41 113.66) (width 0.4) (layer "B.Cu") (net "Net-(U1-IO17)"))
 (segment (start 198.25 112.25) (end 196 114.5) (width 0.4) (layer "B.Cu") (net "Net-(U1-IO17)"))
 (segment (start 166.41 113.66) (end 167.25 114.5) (width 0.4) (layer "B.Cu") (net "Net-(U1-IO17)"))
 (segment (start 140.87 111.12) (end 139.85 111.12) (width 0.4) (layer "B.Cu") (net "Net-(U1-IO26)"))
 (segment (start 145.75 116) (end 140.87 111.12) (width 0.4) (layer "B.Cu") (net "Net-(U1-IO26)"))
 (segment (start 145.75 142) (end 145.75 116) (width 0.4) (layer "B.Cu") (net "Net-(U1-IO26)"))
 (segment (start 147.79 144.04) (end 145.75 142) (width 0.4) (layer "B.Cu") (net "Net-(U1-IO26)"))
 (segment (start 183.25 144.04) (end 147.79 144.04) (width 0.4) (layer "B.Cu") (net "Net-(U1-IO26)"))
 (segment (start 150.75 141.5) (end 148.75 139.5) (width 0.4) (layer "B.Cu") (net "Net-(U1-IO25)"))
 (segment (start 183.25 141.5) (end 150.75 141.5) (width 0.4) (layer "B.Cu") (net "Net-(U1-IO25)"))
 (segment (start 148.75 139.5) (end 148.75 115.5) (width 0.4) (layer "B.Cu") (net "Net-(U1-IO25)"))
 (segment (start 148.75 115.5) (end 141.83 108.58) (width 0.4) (layer "B.Cu") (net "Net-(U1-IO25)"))
 (segment (start 141.83 108.58) (end 139.85 108.58) (width 0.4) (layer "B.Cu") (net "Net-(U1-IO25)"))
 (segment (start 142.75 144) (end 142.75 115.5) (width 0.4) (layer "B.Cu") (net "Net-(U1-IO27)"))
 (segment (start 142.75 115.5) (end 140.91 113.66) (width 0.4) (layer "B.Cu") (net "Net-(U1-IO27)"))
 (segment (start 145.33 146.58) (end 142.75 144) (width 0.4) (layer "B.Cu") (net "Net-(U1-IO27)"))
 (segment (start 183.25 146.58) (end 145.33 146.58) (width 0.4) (layer "B.Cu") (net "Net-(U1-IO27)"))
 (segment (start 140.91 113.66) (end 139.85 113.66) (width 0.4) (layer "B.Cu") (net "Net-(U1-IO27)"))
 (segment (start 132.04 106.04) (end 139.85 106.04) (width 0.4) (layer "B.Cu") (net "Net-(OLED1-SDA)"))
 (segment (start 131.75 106) (end 132 106) (width 0.4) (layer "B.Cu") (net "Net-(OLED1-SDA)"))
 (segment (start 132 106) (end 132.04 106.04) (width 0.4) (layer "B.Cu") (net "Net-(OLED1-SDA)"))
 (segment (start 113.75 124) (end 131.75 106) (width 0.4) (layer "B.Cu") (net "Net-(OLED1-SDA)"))
 (segment (start 111.21 124) (end 111.21 127.21) (width 0.4) (layer "B.Cu") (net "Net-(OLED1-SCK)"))
 (segment (start 111.21 127.21) (end 112 128) (width 0.4) (layer "B.Cu") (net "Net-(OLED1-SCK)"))
 (segment (start 118.18 123.82) (end 139.85 123.82) (width 0.4) (layer "B.Cu") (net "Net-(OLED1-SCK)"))
 (segment (start 117 127) (end 117 125) (width 0.4) (layer "B.Cu") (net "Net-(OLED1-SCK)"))
 (segment (start 117 125) (end 118.18 123.82) (width 0.4) (layer "B.Cu") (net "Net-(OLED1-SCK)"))
 (segment (start 112 128) (end 116 128) (width 0.4) (layer "B.Cu") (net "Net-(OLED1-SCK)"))
 (segment (start 116 128) (end 117 127) (width 0.4) (layer "B.Cu") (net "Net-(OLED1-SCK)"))
 (segment (start 162.5 138.75) (end 163.5 138.75) (width 2) (layer "F.Cu") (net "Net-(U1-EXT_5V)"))
 (segment (start 165 140.25) (end 165 149) (width 2) (layer "F.Cu") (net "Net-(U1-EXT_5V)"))
 (segment (start 163.5 138.75) (end 165 140.25) (width 2) (layer "F.Cu") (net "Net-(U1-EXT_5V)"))
 (segment (start 165 149) (end 164.25 149.75) (width 2) (layer "F.Cu") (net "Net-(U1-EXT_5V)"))
 (segment (start 164.25 149.75) (end 162.75 149.75) (width 2) (layer "F.Cu") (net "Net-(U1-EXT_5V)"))
 (via (at 162.5 138.75) (size 0.6) (drill 0.3) (layers "F.Cu" "B.Cu") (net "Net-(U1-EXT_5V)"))
 (via (at 162.75 149.75) (size 0.6) (drill 0.3) (layers "F.Cu" "B.Cu") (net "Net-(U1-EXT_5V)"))
 (segment (start 157 75) (end 208.25 75) (width 2) (layer "B.Cu") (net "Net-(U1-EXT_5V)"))
 (segment (start 211.5 71.75) (end 211.5 66.25) (width 2) (layer "B.Cu") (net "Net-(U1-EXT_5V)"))
 (segment (start 139.85 145.35) (end 139.85 133.98) (width 2) (layer "B.Cu") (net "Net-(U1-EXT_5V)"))
 (segment (start 208.25 75) (end 211.5 71.75) (width 2) (layer "B.Cu") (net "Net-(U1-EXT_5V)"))
 (segment (start 162.5 138.75) (end 158 138.75) (width 2) (layer "B.Cu") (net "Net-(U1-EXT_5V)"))
 (segment (start 152.75 133.5) (end 152.75 79.25) (width 2) (layer "B.Cu") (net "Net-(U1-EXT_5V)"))
 (segment (start 211.5 66.25) (end 209.75 64.5) (width 2) (layer "B.Cu") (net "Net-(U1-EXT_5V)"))
 (segment (start 152.75 79.25) (end 157 75) (width 2) (layer "B.Cu") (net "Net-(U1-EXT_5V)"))
 (segment (start 158 138.75) (end 152.75 133.5) (width 2) (layer "B.Cu") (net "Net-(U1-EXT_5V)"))
 (segment (start 144.25 149.75) (end 139.85 145.35) (width 2) (layer "B.Cu") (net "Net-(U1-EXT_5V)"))
 (segment (start 209.75 64.5) (end 204.5 64.5) (width 2) (layer "B.Cu") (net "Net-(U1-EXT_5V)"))
 (segment (start 162.75 149.75) (end 144.25 149.75) (width 2) (layer "B.Cu") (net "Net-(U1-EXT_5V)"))
 (segment (start 167.5 37.5) (end 172.95 42.95) (width 2) (layer "B.Cu") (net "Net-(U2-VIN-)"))
 (segment (start 109.905 67.92) (end 112.58 67.92) (width 2) (layer "B.Cu") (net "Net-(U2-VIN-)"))
 (segment (start 115.75 64.75) (end 115.75 37.5) (width 2) (layer "B.Cu") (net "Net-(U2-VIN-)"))
 (segment (start 112.58 67.92) (end 115.75 64.75) (width 2) (layer "B.Cu") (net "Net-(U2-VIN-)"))
 (segment (start 172.95 42.95) (end 172.95 57.3) (width 2) (layer "B.Cu") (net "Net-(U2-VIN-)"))
 (segment (start 115.75 37.5) (end 167.5 37.5) (width 2) (layer "B.Cu") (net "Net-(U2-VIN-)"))
 (segment (start 172.95 68.45) (end 172.95 64.5) (width 2) (layer "B.Cu") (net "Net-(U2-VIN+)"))
 (segment (start 169.75 71.5) (end 172.875 68.375) (width 2) (layer "B.Cu") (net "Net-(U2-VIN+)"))
 (segment (start 107.19 53.56) (end 103.5 57.25) (width 2) (layer "B.Cu") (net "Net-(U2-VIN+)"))
 (segment (start 103.5 69.5) (end 105.5 71.5) (width 2) (layer "B.Cu") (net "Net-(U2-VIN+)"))
 (segment (start 103.5 57.25) (end 103.5 69.5) (width 2) (layer "B.Cu") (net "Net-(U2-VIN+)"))
 (segment (start 172.875 68.375) (end 172.95 68.45) (width 2) (layer "B.Cu") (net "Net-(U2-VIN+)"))
 (segment (start 105.5 71.5) (end 169.75 71.5) (width 2) (layer "B.Cu") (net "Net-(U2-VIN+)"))
 (segment (start 109.905 53.56) (end 107.19 53.56) (width 2) (layer "B.Cu") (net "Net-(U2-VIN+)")))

